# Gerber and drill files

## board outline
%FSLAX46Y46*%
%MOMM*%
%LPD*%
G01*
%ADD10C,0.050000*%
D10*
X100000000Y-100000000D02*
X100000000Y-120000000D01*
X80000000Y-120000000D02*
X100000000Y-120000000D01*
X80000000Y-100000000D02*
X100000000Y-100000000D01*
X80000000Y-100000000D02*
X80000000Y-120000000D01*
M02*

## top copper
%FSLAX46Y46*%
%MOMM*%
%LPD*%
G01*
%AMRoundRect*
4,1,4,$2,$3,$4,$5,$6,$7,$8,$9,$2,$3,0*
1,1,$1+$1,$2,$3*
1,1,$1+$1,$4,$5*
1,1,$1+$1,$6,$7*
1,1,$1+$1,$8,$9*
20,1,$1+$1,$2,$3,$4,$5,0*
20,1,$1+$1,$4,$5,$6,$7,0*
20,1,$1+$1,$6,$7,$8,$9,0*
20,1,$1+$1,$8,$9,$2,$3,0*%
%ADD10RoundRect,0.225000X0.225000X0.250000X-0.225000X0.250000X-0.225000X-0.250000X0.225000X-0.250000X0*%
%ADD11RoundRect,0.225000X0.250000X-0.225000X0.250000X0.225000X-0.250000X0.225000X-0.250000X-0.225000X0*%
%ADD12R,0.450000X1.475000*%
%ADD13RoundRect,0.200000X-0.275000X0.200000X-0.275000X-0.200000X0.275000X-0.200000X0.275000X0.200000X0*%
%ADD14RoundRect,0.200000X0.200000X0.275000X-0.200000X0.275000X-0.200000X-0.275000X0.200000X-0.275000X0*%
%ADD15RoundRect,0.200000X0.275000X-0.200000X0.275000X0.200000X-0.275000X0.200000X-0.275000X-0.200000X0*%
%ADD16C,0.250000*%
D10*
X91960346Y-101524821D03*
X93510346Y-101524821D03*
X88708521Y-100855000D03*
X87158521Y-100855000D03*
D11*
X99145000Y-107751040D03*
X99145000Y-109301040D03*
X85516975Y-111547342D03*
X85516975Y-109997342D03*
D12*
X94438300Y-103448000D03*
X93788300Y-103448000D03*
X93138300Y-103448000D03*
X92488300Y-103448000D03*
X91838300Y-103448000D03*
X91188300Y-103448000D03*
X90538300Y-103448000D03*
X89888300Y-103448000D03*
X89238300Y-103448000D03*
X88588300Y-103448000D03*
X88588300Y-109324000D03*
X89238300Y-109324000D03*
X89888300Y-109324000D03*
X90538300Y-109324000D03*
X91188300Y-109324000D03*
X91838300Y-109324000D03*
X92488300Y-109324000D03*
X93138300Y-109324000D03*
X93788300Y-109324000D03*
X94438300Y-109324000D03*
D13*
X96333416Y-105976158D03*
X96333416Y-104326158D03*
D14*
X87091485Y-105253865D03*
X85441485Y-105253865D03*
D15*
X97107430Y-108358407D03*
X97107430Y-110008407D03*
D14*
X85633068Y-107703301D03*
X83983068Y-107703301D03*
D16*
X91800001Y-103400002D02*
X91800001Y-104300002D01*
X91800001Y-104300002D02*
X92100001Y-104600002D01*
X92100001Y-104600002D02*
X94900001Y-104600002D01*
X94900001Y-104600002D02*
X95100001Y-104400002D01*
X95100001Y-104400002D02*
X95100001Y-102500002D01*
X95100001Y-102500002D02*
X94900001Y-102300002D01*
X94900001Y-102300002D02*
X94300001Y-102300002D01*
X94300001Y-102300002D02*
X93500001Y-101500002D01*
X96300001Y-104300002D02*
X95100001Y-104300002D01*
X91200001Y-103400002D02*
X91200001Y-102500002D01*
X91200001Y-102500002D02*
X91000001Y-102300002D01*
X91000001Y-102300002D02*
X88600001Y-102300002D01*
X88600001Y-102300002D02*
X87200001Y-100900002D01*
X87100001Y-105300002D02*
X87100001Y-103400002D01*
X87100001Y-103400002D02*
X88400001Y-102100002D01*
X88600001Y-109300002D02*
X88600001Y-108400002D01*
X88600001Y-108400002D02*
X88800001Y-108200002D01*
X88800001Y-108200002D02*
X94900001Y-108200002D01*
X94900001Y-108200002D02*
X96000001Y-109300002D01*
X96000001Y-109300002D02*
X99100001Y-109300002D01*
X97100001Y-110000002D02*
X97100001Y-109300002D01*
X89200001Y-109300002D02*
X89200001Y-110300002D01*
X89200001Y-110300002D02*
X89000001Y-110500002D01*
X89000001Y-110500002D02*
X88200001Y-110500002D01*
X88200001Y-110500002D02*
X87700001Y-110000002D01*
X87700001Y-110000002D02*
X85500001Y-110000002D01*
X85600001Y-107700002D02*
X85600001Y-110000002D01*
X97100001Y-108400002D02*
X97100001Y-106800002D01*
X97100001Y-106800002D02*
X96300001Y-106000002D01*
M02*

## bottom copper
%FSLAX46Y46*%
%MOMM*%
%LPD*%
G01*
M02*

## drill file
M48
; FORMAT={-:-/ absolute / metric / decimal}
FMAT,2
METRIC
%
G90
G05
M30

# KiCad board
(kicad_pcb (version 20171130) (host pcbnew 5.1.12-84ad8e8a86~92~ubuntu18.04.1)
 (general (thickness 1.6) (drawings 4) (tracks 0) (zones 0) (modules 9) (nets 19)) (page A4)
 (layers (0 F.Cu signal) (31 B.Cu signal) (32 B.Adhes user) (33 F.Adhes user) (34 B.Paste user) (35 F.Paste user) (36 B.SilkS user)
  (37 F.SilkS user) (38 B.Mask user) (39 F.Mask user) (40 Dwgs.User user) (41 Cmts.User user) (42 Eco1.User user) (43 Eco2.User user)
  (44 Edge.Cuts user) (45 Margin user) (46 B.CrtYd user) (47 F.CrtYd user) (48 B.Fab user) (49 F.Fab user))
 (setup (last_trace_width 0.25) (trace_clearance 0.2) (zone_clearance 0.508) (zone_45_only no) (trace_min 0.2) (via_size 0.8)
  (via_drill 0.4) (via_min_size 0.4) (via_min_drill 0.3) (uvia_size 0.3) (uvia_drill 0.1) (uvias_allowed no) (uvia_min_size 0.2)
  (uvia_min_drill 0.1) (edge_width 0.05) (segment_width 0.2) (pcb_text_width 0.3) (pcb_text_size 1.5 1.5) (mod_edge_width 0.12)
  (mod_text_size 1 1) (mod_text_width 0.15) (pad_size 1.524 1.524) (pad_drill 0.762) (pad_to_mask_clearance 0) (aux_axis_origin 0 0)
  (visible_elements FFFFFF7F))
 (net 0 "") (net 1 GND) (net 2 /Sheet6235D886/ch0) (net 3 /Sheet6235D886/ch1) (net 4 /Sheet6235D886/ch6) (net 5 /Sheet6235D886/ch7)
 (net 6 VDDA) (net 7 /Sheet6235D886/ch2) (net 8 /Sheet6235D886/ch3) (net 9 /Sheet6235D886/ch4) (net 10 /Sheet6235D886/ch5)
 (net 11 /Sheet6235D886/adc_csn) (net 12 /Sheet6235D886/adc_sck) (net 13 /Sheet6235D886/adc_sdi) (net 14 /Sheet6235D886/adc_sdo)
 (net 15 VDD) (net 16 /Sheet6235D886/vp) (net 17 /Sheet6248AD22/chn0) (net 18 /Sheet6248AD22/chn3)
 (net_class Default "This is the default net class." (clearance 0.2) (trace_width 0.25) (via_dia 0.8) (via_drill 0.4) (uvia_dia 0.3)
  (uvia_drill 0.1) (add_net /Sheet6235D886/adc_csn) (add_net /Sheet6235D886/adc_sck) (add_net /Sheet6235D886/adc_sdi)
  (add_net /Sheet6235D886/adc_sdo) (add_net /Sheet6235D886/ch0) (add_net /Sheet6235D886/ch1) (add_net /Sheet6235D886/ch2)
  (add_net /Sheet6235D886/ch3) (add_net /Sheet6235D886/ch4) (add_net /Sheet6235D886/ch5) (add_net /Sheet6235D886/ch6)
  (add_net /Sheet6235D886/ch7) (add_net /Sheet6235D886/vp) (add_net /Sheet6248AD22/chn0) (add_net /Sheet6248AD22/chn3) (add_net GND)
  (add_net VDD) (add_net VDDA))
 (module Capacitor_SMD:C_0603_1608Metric (layer F.Cu) (at 92.735346 101.524821 180.000000)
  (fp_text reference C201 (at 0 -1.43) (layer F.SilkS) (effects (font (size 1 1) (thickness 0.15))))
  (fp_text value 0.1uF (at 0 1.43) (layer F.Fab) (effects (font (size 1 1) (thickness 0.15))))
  (pad 2 smd roundrect (at 0.775 0 180.000000) (size 0.9 0.95) (layers F.Cu F.Mask F.Paste) (roundrect_rratio 0.25) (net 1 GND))
  (pad 1 smd roundrect (at -0.775 0 180.000000) (size 0.9 0.95) (layers F.Cu F.Mask F.Paste) (roundrect_rratio 0.25)
   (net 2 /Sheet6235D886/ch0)))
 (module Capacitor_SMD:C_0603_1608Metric (layer F.Cu) (at 87.933521 100.855000 180.000000)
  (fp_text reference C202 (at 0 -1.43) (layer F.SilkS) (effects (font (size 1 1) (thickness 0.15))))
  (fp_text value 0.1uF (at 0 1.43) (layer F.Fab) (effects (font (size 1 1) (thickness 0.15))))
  (pad 1 smd roundrect (at -0.775 0 180.000000) (size 0.9 0.95) (layers F.Cu F.Mask F.Paste) (roundrect_rratio 0.25) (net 1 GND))
  (pad 2 smd roundrect (at 0.775 0 180.000000) (size 0.9 0.95) (layers F.Cu F.Mask F.Paste) (roundrect_rratio 0.25)
   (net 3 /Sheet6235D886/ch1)))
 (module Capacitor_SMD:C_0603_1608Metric (layer F.Cu) (at 99.145000 108.526040 90.000000)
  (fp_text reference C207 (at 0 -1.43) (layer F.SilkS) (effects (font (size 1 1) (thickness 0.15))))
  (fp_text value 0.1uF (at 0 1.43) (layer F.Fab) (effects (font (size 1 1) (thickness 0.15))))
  (pad 2 smd roundrect (at 0.775 0 90.000000) (size 0.9 0.95) (layers F.Cu F.Mask F.Paste) (roundrect_rratio 0.25) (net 1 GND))
  (pad 1 smd roundrect (at -0.775 0 90.000000) (size 0.9 0.95) (layers F.Cu F.Mask F.Paste) (roundrect_rratio 0.25)
   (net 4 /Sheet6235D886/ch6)))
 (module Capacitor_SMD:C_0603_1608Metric (layer F.Cu) (at 85.516975 110.772342 90.000000)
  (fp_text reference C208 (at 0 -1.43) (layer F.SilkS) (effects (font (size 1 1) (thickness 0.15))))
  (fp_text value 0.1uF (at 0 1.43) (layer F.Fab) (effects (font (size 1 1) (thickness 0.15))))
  (pad 1 smd roundrect (at -0.775 0 90.000000) (size 0.9 0.95) (layers F.Cu F.Mask F.Paste) (roundrect_rratio 0.25) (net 1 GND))
  (pad 2 smd roundrect (at 0.775 0 90.000000) (size 0.9 0.95) (layers F.Cu F.Mask F.Paste) (roundrect_rratio 0.25)
   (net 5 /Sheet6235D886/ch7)))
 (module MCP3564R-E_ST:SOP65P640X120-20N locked (layer F.Cu) (at 91.513300 106.386000 270.000000)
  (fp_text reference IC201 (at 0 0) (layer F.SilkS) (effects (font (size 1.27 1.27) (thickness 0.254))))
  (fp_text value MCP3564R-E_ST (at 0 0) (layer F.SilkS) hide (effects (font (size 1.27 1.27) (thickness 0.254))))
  (pad 1 smd rect (at -2.938 -2.925) (size 0.45 1.475) (layers F.Cu F.Mask F.Paste) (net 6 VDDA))
  (pad 2 smd rect (at -2.938 -2.275) (size 0.45 1.475) (layers F.Cu F.Mask F.Paste) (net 1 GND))
  (pad 3 smd rect (at -2.938 -1.625) (size 0.45 1.475) (layers F.Cu F.Mask F.Paste) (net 1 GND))
  (pad 4 smd rect (at -2.938 -0.975) (size 0.45 1.475) (layers F.Cu F.Mask F.Paste))
  (pad 5 smd rect (at -2.938 -0.325) (size 0.45 1.475) (layers F.Cu F.Mask F.Paste) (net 2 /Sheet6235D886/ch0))
  (pad 6 smd rect (at -2.938 0.325) (size 0.45 1.475) (layers F.Cu F.Mask F.Paste) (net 3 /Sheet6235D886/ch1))
  (pad 7 smd rect (at -2.938 0.975) (size 0.45 1.475) (layers F.Cu F.Mask F.Paste) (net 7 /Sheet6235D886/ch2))
  (pad 8 smd rect (at -2.938 1.625) (size 0.45 1.475) (layers F.Cu F.Mask F.Paste) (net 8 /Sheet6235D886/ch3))
  (pad 9 smd rect (at -2.938 2.275) (size 0.45 1.475) (layers F.Cu F.Mask F.Paste) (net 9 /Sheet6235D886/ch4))
  (pad 10 smd rect (at -2.938 2.925) (size 0.45 1.475) (layers F.Cu F.Mask F.Paste) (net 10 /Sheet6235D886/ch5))
  (pad 11 smd rect (at 2.938 2.925) (size 0.45 1.475) (layers F.Cu F.Mask F.Paste) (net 4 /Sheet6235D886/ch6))
  (pad 12 smd rect (at 2.938 2.275) (size 0.45 1.475) (layers F.Cu F.Mask F.Paste) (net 5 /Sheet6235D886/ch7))
  (pad 13 smd rect (at 2.938 1.625) (size 0.45 1.475) (layers F.Cu F.Mask F.Paste) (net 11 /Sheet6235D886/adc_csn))
  (pad 14 smd rect (at 2.938 0.975) (size 0.45 1.475) (layers F.Cu F.Mask F.Paste) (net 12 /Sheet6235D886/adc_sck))
  (pad 15 smd rect (at 2.938 0.325) (size 0.45 1.475) (layers F.Cu F.Mask F.Paste) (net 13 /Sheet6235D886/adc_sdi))
  (pad 16 smd rect (at 2.938 -0.325) (size 0.45 1.475) (layers F.Cu F.Mask F.Paste) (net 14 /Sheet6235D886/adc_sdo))
  (pad 17 smd rect (at 2.938 -0.975) (size 0.45 1.475) (layers F.Cu F.Mask F.Paste))
  (pad 18 smd rect (at 2.938 -1.625) (size 0.45 1.475) (layers F.Cu F.Mask F.Paste))
  (pad 19 smd rect (at 2.938 -2.275) (size 0.45 1.475) (layers F.Cu F.Mask F.Paste) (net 1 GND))
  (pad 20 smd rect (at 2.938 -2.925) (size 0.45 1.475) (layers F.Cu F.Mask F.Paste) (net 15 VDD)))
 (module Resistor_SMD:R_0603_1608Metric (layer F.Cu) (at 96.333416 105.151158 270.000000)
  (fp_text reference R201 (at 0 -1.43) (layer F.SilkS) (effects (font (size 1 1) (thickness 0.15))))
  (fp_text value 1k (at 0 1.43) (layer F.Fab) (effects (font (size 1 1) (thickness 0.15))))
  (pad 2 smd roundrect (at 0.825 0 270.000000) (size 0.8 0.95) (layers F.Cu F.Mask F.Paste) (roundrect_rratio 0.25)
   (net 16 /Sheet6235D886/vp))
  (pad 1 smd roundrect (at -0.825 0 270.000000) (size 0.8 0.95) (layers F.Cu F.Mask F.Paste) (roundrect_rratio 0.25)
   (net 2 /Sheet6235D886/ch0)))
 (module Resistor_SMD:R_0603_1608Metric (layer F.Cu) (at 86.266485 105.253865 180.000000)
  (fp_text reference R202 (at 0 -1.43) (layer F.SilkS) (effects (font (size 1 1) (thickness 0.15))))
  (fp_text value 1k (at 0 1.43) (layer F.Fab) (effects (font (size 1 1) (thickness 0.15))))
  (pad 1 smd roundrect (at -0.825 0 180.000000) (size 0.8 0.95) (layers F.Cu F.Mask F.Paste) (roundrect_rratio 0.25)
   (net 3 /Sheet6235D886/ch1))
  (pad 2 smd roundrect (at 0.825 0 180.000000) (size 0.8 0.95) (layers F.Cu F.Mask F.Paste) (roundrect_rratio 0.25)
   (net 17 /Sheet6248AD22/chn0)))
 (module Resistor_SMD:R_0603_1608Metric (layer F.Cu) (at 97.107430 109.183407 90.000000)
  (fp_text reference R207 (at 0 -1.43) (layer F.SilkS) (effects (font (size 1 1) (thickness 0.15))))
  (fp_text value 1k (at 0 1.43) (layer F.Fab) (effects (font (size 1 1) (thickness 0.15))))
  (pad 2 smd roundrect (at 0.825 0 90.000000) (size 0.8 0.95) (layers F.Cu F.Mask F.Paste) (roundrect_rratio 0.25)
   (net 16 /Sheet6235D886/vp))
  (pad 1 smd roundrect (at -0.825 0 90.000000) (size 0.8 0.95) (layers F.Cu F.Mask F.Paste) (roundrect_rratio 0.25)
   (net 4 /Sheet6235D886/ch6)))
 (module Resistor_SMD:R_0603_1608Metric (layer F.Cu) (at 84.808068 107.703301 180.000000)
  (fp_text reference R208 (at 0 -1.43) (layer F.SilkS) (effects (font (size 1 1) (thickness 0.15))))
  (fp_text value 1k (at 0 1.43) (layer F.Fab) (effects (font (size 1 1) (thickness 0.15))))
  (pad 1 smd roundrect (at -0.825 0 180.000000) (size 0.8 0.95) (layers F.Cu F.Mask F.Paste) (roundrect_rratio 0.25)
   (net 5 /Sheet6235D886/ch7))
  (pad 2 smd roundrect (at 0.825 0 180.000000) (size 0.8 0.95) (layers F.Cu F.Mask F.Paste) (roundrect_rratio 0.25)
   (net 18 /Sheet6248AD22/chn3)))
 (gr_line (start 100 100) (end 100 120) (layer Edge.Cuts) (width 0.05))
 (gr_line (start 80 120) (end 100 120) (layer Edge.Cuts) (width 0.05))
 (gr_line (start 80 100) (end 100 100) (layer Edge.Cuts) (width 0.05))
 (gr_line (start 80 100) (end 80 120) (layer Edge.Cuts) (width 0.05))
 (segment (start 91.800001 103.400002) (end 91.800001 104.300002) (width 0.250000) (layer F.Cu) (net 2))
 (segment (start 91.800001 104.300002) (end 92.100001 104.600002) (width 0.250000) (layer F.Cu) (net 2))
 (segment (start 92.100001 104.600002) (end 94.900001 104.600002) (width 0.250000) (layer F.Cu) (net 2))
 (segment (start 94.900001 104.600002) (end 95.100001 104.400002) (width 0.250000) (layer F.Cu) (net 2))
 (segment (start 95.100001 104.400002) (end 95.100001 102.500002) (width 0.250000) (layer F.Cu) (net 2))
 (segment (start 95.100001 102.500002) (end 94.900001 102.300002) (width 0.250000) (layer F.Cu) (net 2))
 (segment (start 94.900001 102.300002) (end 94.300001 102.300002) (width 0.250000) (layer F.Cu) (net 2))
 (segment (start 94.300001 102.300002) (end 93.500001 101.500002) (width 0.250000) (layer F.Cu) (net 2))
 (segment (start 96.300001 104.300002) (end 95.100001 104.300002) (width 0.250000) (layer F.Cu) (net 2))
 (segment (start 91.200001 103.400002) (end 91.200001 102.500002) (width 0.250000) (layer F.Cu) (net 3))
 (segment (start 91.200001 102.500002) (end 91.000001 102.300002) (width 0.250000) (layer F.Cu) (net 3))
 (segment (start 91.000001 102.300002) (end 88.600001 102.300002) (width 0.250000) (layer F.Cu) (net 3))
 (segment (start 88.600001 102.300002) (end 87.200001 100.900002) (width 0.250000) (layer F.Cu) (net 3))
 (segment (start 87.100001 105.300002) (end 87.100001 103.400002) (width 0.250000) (layer F.Cu) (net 3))
 (segment (start 87.100001 103.400002) (end 88.400001 102.100002) (width 0.250000) (layer F.Cu) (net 3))
 (segment (start 88.600001 109.300002) (end 88.600001 108.400002) (width 0.250000) (layer F.Cu) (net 4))
 (segment (start 88.600001 108.400002) (end 88.800001 108.200002) (width 0.250000) (layer F.Cu) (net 4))
 (segment (start 88.800001 108.200002) (end 94.900001 108.200002) (width 0.250000) (layer F.Cu) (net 4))
 (segment (start 94.900001 108.200002) (end 96.000001 109.300002) (width 0.250000) (layer F.Cu) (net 4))
 (segment (start 96.000001 109.300002) (end 99.100001 109.300002) (width 0.250000) (layer F.Cu) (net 4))
 (segment (start 97.100001 110.000002) (end 97.100001 109.300002) (width 0.250000) (layer F.Cu) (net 4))
 (segment (start 89.200001 109.300002) (end 89.200001 110.300002) (width 0.250000) (layer F.Cu) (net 5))
 (segment (start 89.200001 110.300002) (end 89.000001 110.500002) (width 0.250000) (layer F.Cu) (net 5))
 (segment (start 89.000001 110.500002) (end 88.200001 110.500002) (width 0.250000) (layer F.Cu) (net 5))
 (segment (start 88.200001 110.500002) (end 87.700001 110.000002) (width 0.250000) (layer F.Cu) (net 5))
 (segment (start 87.700001 110.000002) (end 85.500001 110.000002) (width 0.250000) (layer F.Cu) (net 5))
 (segment (start 85.600001 107.700002) (end 85.600001 110.000002) (width 0.250000) (layer F.Cu) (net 5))
 (segment (start 97.100001 108.400002) (end 97.100001 106.800002) (width 0.250000) (layer F.Cu) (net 16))
 (segment (start 97.100001 106.800002) (end 96.300001 106.000002) (width 0.250000) (layer F.Cu) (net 16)))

